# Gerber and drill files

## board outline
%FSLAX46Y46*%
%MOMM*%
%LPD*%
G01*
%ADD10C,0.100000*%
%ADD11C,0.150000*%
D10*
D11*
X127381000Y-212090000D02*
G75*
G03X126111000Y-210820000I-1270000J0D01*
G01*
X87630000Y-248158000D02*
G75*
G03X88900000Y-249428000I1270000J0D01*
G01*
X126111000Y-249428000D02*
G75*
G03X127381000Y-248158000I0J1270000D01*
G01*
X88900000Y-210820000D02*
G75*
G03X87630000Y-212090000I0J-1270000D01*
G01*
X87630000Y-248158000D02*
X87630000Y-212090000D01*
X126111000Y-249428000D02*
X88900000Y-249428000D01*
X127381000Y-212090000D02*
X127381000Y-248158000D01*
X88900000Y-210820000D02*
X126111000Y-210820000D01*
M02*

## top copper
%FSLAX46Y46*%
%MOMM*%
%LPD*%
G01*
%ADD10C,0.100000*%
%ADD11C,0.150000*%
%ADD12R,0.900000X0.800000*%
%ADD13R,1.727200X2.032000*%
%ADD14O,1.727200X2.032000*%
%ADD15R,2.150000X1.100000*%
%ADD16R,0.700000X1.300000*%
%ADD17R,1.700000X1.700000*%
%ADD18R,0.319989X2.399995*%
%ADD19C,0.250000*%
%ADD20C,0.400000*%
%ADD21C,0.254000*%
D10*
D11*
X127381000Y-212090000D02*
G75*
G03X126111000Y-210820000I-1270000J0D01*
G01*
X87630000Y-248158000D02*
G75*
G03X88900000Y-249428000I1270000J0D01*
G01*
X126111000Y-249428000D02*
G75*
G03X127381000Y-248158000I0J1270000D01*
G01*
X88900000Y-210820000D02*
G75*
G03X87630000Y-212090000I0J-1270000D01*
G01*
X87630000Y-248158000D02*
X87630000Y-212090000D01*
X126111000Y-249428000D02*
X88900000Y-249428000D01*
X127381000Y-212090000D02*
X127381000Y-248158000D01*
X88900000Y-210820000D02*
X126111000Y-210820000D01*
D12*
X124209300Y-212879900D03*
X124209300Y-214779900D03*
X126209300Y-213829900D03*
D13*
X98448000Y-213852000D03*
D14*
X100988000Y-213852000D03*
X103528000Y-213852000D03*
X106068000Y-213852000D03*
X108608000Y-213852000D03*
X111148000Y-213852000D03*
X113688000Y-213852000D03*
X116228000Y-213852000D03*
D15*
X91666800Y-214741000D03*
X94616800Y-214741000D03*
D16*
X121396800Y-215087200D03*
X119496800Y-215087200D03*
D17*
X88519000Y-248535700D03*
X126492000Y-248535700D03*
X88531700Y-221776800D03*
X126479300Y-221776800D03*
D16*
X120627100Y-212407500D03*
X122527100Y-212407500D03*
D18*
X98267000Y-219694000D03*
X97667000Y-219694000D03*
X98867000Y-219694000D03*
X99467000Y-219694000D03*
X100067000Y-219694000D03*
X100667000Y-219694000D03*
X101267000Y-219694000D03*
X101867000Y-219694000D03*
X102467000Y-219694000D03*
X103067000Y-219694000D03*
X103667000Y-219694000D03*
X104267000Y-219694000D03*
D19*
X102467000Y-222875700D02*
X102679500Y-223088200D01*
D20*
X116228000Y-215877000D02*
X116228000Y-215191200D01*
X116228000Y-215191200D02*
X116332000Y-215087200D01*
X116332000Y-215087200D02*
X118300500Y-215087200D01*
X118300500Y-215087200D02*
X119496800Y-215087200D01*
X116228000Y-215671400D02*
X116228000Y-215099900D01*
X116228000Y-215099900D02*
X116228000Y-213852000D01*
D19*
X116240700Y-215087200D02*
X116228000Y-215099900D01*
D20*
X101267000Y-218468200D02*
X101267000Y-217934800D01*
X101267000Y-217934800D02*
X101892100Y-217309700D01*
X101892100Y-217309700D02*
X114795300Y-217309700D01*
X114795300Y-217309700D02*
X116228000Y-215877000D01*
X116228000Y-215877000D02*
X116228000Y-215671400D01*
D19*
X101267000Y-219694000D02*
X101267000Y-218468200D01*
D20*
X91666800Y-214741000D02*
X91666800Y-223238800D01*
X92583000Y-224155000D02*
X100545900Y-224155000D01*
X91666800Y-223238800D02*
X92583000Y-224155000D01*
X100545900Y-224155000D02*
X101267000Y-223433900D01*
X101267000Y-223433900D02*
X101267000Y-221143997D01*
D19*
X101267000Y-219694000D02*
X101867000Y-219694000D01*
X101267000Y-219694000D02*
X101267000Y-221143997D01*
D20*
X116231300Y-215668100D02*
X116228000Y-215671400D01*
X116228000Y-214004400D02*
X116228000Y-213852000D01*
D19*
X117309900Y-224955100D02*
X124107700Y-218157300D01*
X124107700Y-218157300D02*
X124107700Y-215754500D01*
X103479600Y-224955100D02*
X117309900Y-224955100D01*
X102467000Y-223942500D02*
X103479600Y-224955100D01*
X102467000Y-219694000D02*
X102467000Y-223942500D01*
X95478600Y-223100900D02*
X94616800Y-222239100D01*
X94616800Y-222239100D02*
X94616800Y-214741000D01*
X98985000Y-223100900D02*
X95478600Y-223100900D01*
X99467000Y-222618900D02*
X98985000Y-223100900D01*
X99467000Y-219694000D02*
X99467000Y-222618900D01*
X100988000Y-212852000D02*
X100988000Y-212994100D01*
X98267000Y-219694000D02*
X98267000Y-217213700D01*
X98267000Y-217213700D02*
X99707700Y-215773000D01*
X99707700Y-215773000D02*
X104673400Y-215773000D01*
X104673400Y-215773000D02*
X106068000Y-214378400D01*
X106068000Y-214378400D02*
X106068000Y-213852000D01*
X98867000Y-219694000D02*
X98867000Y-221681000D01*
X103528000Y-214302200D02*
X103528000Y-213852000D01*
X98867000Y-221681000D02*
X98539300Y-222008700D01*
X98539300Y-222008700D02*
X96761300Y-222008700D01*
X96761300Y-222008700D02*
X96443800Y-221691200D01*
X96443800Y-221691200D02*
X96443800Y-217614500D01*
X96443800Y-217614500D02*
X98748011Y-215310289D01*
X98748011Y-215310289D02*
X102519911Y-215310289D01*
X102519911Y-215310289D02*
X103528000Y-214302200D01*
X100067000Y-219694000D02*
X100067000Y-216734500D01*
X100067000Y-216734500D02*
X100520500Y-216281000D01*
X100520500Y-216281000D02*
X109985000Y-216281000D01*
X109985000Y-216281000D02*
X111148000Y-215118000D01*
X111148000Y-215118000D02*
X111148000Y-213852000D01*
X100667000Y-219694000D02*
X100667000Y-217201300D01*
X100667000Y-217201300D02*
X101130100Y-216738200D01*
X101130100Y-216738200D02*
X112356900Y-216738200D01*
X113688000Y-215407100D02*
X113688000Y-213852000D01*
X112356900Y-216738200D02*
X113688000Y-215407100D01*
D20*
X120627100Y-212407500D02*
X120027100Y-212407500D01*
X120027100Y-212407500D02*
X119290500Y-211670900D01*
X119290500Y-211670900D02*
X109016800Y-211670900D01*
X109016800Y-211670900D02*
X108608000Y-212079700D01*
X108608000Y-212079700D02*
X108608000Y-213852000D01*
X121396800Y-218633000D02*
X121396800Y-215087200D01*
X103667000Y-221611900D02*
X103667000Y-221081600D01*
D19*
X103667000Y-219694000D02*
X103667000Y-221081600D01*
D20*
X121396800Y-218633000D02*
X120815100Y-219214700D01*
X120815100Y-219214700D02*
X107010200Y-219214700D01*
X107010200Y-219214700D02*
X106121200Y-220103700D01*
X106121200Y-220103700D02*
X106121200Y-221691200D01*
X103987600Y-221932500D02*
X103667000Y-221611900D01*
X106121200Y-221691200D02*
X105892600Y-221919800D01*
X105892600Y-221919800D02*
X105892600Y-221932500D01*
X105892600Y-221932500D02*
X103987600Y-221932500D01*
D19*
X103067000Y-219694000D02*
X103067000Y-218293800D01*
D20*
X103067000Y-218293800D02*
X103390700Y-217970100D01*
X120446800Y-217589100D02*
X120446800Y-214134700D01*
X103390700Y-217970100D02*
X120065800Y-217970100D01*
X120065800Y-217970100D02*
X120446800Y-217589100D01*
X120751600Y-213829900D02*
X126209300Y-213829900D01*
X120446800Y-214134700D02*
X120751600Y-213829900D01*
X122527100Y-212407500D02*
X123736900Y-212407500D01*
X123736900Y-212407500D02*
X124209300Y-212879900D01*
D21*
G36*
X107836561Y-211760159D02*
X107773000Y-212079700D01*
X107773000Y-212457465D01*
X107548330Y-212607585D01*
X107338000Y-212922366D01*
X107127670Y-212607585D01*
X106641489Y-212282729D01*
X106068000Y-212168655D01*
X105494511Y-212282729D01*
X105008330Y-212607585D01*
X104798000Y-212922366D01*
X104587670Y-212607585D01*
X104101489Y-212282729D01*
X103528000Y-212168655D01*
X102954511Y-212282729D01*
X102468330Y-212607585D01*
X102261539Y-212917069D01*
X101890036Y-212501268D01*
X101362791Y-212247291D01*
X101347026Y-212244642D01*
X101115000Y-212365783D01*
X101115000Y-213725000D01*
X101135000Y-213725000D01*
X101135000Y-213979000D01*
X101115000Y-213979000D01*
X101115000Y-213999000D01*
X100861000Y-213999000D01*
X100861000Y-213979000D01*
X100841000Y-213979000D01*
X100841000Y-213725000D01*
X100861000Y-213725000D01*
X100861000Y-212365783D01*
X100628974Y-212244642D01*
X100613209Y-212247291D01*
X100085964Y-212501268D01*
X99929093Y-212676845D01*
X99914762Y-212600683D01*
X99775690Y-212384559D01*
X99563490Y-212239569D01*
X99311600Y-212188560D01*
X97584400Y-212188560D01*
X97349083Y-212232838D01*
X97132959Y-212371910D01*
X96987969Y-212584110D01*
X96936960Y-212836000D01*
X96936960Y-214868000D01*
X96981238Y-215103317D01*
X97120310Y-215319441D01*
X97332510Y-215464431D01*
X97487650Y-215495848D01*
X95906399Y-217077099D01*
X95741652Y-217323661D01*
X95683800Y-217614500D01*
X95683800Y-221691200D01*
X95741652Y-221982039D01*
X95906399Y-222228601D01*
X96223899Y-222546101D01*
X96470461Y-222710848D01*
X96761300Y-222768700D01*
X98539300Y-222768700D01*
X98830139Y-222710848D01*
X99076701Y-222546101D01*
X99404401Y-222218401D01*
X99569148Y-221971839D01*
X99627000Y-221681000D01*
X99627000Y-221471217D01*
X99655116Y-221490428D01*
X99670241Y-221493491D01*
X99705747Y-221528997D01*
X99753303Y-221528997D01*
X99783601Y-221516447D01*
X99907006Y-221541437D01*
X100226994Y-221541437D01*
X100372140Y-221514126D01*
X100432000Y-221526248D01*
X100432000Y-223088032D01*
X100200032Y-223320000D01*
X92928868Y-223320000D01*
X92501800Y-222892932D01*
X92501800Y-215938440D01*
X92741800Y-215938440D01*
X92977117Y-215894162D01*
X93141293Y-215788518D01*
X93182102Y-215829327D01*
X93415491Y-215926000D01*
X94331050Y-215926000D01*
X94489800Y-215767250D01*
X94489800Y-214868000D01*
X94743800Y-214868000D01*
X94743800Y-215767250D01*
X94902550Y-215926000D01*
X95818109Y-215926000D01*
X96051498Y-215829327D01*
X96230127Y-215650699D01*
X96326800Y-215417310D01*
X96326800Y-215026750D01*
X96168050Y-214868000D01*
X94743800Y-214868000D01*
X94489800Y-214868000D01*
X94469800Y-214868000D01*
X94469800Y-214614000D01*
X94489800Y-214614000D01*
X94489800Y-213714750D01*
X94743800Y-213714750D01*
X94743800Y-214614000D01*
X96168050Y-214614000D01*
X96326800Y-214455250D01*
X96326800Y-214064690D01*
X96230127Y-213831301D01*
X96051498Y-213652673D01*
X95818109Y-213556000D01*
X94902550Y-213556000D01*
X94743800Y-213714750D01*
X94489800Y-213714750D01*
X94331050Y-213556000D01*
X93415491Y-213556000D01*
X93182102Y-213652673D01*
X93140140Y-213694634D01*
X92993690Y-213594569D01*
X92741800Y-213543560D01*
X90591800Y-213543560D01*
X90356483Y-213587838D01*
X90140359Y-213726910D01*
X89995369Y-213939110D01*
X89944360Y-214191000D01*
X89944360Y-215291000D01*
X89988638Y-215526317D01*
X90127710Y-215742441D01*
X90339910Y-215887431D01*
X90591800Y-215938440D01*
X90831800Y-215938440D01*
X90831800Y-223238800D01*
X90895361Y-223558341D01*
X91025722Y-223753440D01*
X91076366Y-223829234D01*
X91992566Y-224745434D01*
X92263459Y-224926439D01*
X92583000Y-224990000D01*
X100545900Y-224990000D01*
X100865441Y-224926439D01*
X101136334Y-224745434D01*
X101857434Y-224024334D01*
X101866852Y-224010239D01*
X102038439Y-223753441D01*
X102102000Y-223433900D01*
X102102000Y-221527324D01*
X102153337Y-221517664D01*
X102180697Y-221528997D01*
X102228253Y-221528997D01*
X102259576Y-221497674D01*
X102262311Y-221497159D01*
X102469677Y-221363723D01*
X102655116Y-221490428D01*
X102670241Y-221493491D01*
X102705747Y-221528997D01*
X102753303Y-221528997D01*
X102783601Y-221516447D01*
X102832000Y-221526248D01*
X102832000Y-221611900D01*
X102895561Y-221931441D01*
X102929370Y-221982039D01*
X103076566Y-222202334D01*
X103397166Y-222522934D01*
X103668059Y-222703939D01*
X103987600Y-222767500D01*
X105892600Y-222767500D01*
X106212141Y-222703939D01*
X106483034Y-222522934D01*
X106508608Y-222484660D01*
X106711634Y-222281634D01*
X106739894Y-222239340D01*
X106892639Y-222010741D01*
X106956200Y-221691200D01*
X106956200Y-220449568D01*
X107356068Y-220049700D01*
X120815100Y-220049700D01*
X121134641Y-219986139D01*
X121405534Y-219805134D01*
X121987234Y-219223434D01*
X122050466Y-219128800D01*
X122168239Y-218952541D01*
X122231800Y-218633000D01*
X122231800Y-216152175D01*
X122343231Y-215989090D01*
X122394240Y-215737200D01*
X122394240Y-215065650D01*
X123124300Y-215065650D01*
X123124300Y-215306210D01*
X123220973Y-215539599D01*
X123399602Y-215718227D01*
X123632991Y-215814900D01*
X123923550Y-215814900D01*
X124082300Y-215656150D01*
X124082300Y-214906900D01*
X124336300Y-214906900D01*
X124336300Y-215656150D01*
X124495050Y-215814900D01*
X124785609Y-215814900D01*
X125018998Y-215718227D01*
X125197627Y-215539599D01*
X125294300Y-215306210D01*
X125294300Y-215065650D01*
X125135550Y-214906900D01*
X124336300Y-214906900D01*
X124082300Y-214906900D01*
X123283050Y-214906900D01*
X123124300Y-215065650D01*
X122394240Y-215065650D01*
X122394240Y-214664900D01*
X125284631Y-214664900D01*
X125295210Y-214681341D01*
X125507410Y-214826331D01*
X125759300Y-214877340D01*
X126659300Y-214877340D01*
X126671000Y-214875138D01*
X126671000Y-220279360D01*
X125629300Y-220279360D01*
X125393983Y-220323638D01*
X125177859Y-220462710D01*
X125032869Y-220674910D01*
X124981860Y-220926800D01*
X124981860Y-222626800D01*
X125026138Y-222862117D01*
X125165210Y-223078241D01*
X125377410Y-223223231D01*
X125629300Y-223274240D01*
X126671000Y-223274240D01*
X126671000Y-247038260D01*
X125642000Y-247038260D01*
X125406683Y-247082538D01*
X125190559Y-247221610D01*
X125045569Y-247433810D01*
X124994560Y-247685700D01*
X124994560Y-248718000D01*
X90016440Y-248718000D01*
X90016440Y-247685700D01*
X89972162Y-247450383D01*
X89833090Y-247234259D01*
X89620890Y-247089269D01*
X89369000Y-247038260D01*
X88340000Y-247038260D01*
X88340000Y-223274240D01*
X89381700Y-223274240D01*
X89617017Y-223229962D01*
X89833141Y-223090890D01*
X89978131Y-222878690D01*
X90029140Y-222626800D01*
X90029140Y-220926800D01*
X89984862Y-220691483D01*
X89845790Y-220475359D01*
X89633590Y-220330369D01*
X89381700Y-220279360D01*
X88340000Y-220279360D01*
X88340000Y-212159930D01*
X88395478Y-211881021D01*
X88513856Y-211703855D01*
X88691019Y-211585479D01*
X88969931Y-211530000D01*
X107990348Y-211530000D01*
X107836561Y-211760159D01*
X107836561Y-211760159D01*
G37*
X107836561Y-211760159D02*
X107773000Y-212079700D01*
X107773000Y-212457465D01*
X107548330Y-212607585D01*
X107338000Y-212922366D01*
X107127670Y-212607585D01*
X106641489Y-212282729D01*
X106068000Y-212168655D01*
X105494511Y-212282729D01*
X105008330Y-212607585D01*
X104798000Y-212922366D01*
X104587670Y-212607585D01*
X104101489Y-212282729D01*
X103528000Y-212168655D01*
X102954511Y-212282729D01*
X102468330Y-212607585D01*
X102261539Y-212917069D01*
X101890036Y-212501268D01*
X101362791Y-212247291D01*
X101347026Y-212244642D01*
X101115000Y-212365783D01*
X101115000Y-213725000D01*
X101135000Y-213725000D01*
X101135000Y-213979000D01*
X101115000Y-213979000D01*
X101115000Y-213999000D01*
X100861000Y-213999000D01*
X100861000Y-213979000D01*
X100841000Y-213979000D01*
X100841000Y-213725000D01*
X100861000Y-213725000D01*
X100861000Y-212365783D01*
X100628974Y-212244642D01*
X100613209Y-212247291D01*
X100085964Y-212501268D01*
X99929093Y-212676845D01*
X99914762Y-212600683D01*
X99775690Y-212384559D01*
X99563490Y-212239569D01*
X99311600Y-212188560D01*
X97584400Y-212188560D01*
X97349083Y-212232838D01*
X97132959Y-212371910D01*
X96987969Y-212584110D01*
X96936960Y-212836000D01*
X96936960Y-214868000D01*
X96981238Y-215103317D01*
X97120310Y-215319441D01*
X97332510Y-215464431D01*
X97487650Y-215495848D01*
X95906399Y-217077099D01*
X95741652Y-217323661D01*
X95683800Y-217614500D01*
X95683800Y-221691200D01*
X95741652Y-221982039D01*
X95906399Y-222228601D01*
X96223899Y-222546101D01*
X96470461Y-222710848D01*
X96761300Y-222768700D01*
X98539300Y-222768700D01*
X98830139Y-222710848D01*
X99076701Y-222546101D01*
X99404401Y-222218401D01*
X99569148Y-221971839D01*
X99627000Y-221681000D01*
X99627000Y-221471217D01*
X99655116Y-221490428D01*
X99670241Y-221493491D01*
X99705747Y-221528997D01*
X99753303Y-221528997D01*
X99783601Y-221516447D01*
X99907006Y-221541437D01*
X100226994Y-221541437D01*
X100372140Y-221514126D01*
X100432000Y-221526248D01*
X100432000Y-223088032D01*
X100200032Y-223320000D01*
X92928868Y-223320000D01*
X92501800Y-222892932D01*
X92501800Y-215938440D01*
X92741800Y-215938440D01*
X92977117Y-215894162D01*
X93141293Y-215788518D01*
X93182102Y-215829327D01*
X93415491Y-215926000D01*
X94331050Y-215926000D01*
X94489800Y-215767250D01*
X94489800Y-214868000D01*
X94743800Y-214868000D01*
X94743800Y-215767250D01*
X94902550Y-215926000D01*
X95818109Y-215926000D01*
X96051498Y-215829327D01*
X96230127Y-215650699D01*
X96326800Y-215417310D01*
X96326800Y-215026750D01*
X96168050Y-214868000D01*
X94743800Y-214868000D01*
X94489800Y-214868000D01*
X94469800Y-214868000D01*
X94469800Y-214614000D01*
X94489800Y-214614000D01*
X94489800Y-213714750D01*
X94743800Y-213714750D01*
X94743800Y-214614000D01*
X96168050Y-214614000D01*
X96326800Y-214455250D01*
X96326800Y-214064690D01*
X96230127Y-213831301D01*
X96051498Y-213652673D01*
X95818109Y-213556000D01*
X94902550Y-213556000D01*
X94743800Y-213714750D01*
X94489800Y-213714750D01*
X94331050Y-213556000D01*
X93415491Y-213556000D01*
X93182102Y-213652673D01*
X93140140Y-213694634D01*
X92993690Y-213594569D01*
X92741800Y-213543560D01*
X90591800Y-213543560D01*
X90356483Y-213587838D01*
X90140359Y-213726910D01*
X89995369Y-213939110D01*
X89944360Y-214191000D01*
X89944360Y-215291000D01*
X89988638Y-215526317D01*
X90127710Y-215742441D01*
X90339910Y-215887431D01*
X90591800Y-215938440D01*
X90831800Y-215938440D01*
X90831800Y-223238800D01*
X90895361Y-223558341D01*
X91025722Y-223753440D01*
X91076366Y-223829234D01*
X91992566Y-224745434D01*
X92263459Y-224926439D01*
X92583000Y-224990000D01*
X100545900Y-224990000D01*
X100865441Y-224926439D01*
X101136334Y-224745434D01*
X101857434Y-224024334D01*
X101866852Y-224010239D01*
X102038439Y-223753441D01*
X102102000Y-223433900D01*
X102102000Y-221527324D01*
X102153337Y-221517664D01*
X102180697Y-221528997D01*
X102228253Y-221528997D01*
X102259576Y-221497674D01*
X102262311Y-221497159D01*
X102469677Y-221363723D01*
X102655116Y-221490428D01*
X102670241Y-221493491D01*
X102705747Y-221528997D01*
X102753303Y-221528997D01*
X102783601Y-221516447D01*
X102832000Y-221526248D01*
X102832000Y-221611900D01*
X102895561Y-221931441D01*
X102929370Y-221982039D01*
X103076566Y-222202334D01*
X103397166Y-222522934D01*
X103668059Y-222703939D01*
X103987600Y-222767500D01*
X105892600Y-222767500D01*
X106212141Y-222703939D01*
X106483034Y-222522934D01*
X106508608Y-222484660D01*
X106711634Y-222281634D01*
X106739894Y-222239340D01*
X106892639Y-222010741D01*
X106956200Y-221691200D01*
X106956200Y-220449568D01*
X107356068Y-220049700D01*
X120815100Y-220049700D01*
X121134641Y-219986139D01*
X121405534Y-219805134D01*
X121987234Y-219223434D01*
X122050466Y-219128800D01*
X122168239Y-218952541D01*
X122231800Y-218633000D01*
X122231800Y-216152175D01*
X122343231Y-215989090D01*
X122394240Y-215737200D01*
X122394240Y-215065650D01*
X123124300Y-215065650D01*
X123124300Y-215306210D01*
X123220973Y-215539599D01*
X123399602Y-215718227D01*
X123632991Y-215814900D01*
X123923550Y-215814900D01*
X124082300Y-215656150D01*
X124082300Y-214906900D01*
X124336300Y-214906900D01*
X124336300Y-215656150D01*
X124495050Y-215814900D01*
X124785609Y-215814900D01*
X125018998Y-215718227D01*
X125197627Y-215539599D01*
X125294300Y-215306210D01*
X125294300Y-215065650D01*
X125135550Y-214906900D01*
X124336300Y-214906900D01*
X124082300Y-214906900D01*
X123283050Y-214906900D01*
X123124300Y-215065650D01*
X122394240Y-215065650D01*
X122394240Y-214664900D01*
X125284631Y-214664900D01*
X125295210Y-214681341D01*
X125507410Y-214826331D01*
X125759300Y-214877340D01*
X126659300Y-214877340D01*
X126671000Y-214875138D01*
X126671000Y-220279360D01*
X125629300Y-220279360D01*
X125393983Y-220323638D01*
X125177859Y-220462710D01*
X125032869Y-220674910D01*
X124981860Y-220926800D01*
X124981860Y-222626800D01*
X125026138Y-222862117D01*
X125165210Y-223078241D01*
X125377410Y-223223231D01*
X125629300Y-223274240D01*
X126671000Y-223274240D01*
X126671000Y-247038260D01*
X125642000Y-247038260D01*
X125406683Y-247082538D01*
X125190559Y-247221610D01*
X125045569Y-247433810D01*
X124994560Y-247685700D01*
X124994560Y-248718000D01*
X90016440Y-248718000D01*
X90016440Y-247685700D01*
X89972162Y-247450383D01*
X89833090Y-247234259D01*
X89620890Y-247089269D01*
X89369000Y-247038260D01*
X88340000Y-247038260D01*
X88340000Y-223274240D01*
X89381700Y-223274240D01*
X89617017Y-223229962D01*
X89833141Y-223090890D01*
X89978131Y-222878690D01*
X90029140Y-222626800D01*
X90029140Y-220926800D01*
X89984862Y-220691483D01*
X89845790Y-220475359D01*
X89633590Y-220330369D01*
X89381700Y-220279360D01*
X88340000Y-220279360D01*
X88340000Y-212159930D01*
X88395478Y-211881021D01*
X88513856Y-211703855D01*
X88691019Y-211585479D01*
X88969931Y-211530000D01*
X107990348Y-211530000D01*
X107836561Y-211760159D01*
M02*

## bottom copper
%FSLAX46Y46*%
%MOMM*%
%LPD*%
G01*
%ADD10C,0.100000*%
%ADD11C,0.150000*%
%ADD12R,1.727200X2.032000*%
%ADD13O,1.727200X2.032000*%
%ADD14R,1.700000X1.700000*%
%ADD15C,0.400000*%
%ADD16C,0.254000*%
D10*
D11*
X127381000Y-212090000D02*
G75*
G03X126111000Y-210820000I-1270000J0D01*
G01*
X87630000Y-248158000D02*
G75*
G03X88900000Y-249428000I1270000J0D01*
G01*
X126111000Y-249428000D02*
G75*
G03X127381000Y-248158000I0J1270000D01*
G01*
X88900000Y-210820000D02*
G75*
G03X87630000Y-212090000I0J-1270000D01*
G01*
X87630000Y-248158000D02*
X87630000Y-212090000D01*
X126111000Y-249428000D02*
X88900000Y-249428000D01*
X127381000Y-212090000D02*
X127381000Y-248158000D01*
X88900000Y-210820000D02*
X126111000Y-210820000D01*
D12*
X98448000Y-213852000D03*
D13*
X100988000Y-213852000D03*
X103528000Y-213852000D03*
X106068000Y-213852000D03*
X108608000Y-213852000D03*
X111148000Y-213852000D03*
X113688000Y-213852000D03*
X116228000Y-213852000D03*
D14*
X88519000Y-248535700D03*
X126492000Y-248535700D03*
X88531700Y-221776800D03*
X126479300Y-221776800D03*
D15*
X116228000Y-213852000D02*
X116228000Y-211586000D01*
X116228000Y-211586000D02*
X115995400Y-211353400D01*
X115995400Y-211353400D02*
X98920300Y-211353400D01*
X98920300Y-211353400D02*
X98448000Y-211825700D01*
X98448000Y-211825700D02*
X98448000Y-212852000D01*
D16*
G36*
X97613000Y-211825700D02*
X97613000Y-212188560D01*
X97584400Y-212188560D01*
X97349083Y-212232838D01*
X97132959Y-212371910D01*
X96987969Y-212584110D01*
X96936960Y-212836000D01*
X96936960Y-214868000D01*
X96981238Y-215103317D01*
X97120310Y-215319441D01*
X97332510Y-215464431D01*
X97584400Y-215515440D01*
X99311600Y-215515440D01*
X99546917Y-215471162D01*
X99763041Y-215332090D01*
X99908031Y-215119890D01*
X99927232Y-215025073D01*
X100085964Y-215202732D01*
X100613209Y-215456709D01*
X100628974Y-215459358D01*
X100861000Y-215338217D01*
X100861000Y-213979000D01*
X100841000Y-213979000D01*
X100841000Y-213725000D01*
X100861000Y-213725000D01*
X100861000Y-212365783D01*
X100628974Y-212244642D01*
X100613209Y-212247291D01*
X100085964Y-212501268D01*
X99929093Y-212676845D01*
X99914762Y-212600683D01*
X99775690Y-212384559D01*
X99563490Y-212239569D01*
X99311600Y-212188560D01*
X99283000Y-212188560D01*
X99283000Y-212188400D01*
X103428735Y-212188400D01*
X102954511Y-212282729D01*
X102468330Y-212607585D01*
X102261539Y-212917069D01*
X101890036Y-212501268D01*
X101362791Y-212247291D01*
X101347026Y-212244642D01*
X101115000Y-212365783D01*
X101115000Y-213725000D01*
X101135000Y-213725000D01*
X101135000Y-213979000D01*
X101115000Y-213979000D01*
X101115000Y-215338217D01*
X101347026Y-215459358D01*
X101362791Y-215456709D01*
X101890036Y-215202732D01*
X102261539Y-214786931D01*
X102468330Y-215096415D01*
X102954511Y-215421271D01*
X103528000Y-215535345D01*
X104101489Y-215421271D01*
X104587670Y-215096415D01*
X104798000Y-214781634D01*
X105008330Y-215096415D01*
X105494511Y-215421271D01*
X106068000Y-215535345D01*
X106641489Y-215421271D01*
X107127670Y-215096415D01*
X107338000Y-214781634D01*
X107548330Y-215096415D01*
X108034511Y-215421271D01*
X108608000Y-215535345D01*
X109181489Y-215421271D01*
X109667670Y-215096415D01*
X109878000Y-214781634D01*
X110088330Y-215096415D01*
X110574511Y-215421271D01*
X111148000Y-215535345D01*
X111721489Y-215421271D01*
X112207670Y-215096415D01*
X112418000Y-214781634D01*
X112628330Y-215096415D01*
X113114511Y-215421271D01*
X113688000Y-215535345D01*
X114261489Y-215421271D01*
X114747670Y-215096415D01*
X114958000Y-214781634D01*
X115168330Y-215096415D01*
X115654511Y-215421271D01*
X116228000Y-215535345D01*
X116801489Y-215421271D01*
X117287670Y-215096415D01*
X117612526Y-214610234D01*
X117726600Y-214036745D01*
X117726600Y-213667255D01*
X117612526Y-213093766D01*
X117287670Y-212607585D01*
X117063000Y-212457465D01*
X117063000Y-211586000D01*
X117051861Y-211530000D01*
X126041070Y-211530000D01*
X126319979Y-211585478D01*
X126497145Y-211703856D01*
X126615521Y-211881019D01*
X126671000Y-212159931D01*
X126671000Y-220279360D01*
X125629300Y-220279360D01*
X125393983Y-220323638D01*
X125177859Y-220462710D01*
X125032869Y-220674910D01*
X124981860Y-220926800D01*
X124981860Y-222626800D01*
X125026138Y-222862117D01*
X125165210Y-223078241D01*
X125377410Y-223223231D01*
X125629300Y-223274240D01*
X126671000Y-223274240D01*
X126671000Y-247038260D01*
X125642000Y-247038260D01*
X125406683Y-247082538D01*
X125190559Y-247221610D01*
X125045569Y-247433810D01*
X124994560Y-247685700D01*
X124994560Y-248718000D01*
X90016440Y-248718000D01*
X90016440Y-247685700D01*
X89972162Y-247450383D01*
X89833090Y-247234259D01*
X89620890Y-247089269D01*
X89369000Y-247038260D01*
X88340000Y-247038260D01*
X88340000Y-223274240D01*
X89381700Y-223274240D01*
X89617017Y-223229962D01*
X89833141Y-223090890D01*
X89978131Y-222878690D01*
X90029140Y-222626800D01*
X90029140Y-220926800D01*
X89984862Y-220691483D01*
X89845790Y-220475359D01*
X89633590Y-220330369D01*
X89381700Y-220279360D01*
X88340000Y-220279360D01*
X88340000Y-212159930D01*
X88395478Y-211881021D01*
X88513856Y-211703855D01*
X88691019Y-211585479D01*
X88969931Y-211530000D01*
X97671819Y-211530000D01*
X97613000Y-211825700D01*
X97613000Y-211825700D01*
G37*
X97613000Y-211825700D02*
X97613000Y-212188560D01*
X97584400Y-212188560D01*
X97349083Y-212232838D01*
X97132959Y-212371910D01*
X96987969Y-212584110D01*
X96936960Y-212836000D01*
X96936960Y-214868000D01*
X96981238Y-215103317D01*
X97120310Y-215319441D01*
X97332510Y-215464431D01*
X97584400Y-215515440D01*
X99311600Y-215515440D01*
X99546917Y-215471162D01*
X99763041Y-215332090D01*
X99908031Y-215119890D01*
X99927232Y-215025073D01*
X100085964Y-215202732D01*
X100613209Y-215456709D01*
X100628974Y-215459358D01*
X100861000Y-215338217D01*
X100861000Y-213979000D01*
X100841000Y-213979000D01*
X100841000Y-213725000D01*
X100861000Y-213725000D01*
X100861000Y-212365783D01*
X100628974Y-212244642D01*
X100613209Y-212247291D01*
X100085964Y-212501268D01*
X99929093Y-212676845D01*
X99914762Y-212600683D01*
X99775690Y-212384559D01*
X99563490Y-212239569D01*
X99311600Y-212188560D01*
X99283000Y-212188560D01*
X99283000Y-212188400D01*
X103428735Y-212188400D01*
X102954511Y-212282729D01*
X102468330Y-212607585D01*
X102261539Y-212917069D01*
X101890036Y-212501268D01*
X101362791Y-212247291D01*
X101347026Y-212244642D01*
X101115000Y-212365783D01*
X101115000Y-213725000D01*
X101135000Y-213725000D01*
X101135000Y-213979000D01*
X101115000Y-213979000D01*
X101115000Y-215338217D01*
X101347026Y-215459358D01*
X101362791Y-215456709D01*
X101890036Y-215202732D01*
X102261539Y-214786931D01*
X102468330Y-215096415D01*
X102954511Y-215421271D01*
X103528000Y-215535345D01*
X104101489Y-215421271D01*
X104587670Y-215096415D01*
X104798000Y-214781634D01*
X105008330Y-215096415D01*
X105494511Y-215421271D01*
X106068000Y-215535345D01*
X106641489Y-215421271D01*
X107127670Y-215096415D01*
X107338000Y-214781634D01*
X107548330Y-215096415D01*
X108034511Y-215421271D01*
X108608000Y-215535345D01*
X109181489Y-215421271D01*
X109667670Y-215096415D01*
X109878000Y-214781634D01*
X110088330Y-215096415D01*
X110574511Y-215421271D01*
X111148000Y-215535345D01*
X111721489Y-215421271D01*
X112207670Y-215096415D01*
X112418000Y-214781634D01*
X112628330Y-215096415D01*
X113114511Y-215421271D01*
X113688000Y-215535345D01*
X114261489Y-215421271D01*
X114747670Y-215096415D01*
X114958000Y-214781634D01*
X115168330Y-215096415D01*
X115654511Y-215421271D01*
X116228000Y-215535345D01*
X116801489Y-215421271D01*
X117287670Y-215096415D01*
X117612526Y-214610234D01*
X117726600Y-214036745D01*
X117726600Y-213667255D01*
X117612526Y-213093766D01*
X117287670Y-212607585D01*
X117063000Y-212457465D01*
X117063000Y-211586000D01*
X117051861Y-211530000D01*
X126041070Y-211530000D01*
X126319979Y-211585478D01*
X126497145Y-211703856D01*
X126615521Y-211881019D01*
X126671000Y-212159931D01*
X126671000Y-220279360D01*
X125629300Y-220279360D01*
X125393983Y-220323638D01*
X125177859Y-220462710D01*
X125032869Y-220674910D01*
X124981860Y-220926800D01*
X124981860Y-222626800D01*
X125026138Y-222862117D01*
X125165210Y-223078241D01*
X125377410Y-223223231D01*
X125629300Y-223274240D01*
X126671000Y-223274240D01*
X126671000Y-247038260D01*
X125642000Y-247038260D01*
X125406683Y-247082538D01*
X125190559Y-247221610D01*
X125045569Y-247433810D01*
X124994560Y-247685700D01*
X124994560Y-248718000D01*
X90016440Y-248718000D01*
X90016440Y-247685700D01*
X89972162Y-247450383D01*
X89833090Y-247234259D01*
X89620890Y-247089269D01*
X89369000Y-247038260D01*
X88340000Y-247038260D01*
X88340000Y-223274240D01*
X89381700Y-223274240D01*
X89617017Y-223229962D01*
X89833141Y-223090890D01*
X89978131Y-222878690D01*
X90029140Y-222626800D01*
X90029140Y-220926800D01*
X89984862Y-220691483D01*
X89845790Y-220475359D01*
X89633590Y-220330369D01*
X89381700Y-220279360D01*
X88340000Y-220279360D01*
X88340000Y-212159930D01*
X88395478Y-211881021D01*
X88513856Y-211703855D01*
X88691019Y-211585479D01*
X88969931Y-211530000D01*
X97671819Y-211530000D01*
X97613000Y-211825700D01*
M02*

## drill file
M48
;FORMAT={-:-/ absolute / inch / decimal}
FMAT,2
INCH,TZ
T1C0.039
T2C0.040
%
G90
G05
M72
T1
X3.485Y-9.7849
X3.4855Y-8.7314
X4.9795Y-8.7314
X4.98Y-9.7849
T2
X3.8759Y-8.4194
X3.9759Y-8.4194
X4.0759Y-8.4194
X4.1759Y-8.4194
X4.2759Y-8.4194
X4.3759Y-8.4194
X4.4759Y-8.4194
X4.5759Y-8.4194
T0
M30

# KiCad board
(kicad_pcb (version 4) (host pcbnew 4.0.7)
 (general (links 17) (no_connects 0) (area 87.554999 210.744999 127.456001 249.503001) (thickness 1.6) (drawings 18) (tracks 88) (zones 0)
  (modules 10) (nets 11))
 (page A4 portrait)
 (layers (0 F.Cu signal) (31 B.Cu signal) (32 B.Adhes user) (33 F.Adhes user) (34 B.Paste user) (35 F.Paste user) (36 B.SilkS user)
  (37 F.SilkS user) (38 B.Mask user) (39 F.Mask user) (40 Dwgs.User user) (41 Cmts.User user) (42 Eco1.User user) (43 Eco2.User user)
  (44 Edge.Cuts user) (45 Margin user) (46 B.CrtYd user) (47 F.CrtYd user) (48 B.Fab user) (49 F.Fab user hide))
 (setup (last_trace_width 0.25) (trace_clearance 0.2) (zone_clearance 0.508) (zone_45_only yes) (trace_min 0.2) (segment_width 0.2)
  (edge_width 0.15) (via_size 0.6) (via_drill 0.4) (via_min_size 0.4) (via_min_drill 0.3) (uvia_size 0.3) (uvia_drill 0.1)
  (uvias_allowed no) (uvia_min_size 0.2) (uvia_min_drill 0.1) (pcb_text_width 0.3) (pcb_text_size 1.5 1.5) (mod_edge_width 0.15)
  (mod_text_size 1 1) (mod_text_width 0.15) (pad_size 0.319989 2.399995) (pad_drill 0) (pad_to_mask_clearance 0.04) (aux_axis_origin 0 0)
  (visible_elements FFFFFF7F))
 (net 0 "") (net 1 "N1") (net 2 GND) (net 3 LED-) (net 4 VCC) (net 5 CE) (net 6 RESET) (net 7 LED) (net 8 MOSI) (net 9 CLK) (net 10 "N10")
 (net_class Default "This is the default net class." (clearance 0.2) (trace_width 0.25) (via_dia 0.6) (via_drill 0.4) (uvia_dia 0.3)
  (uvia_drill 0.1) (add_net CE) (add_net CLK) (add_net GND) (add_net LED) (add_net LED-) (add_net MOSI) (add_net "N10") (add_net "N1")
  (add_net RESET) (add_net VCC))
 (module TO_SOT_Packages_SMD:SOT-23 (layer F.Cu) (at 125.2093 213.8299)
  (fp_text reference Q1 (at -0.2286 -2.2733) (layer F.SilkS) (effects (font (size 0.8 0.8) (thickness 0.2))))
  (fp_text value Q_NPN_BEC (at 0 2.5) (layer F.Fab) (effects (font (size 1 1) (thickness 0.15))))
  (pad 1 smd rect (at -1 -0.95) (size 0.9 0.8) (layers F.Cu F.Paste F.Mask) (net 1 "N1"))
  (pad 2 smd rect (at -1 0.95) (size 0.9 0.8) (layers F.Cu F.Paste F.Mask) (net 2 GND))
  (pad 3 smd rect (at 1 0) (size 0.9 0.8) (layers F.Cu F.Paste F.Mask) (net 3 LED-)))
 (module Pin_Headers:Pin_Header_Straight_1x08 (layer F.Cu) (at 98.448 213.852 90)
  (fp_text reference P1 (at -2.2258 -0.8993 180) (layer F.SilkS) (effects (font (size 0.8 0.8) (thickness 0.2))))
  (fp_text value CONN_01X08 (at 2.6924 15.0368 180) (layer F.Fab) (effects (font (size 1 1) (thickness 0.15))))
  (pad 1 thru_hole rect (at 0 0 90) (size 2.032 1.7272) (drill 1.016) (layers *.Cu *.Mask F.SilkS) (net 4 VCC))
  (pad 2 thru_hole oval (at 0 2.54 90) (size 2.032 1.7272) (drill 1.016) (layers *.Cu *.Mask F.SilkS) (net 2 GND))
  (pad 3 thru_hole oval (at 0 5.08 90) (size 2.032 1.7272) (drill 1.016) (layers *.Cu *.Mask F.SilkS) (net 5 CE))
  (pad 4 thru_hole oval (at 0 7.62 90) (size 2.032 1.7272) (drill 1.016) (layers *.Cu *.Mask F.SilkS) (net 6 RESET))
  (pad 5 thru_hole oval (at 0 10.16 90) (size 2.032 1.7272) (drill 1.016) (layers *.Cu *.Mask F.SilkS) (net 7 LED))
  (pad 6 thru_hole oval (at 0 12.7 90) (size 2.032 1.7272) (drill 1.016) (layers *.Cu *.Mask F.SilkS) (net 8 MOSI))
  (pad 7 thru_hole oval (at 0 15.24 90) (size 2.032 1.7272) (drill 1.016) (layers *.Cu *.Mask F.SilkS) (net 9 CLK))
  (pad 8 thru_hole oval (at 0 17.78 90) (size 2.032 1.7272) (drill 1.016) (layers *.Cu *.Mask F.SilkS) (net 4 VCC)))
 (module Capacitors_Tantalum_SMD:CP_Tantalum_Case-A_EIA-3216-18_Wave (layer F.Cu) (at 93.1418 214.741)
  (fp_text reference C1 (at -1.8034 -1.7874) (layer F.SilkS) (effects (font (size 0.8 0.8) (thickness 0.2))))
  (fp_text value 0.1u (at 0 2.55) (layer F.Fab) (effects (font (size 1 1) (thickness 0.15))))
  (pad 1 smd rect (at -1.475 0) (size 2.15 1.1) (layers F.Cu F.Paste F.Mask) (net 4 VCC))
  (pad 2 smd rect (at 1.475 0) (size 2.15 1.1) (layers F.Cu F.Paste F.Mask) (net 2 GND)))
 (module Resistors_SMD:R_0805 (layer F.Cu) (at 120.4468 215.0872 180)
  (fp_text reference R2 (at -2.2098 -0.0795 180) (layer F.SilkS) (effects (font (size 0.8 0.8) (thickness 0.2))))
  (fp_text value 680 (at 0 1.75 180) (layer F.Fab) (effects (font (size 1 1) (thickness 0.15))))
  (pad 1 smd rect (at -0.95 0 180) (size 0.7 1.3) (layers F.Cu F.Paste F.Mask) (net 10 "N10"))
  (pad 2 smd rect (at 0.95 0 180) (size 0.7 1.3) (layers F.Cu F.Paste F.Mask) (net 4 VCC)))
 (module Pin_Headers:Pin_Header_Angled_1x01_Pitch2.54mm (layer F.Cu) (at 88.519 248.5357)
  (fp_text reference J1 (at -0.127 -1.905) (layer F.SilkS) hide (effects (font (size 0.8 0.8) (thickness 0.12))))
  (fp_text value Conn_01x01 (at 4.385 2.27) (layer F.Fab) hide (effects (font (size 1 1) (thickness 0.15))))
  (pad 1 thru_hole rect (at 0 0) (size 1.7 1.7) (drill 1) (layers *.Cu *.Mask)))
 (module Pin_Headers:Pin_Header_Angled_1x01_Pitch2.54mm (layer F.Cu) (at 126.492 248.5357 180)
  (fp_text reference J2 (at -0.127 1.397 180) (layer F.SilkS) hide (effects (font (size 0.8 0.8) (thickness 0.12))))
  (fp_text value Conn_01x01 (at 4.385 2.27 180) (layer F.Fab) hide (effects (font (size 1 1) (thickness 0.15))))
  (pad 1 thru_hole rect (at 0 0 180) (size 1.7 1.7) (drill 1) (layers *.Cu *.Mask)))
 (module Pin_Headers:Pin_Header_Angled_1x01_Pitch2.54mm (layer F.Cu) (at 88.5317 221.7768)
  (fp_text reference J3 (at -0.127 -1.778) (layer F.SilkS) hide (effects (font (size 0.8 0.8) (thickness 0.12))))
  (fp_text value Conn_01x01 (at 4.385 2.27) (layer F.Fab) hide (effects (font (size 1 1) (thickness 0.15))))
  (pad 1 thru_hole rect (at 0 0) (size 1.7 1.7) (drill 1) (layers *.Cu *.Mask)))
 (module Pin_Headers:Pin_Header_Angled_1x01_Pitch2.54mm (layer F.Cu) (at 126.4793 221.7768 180)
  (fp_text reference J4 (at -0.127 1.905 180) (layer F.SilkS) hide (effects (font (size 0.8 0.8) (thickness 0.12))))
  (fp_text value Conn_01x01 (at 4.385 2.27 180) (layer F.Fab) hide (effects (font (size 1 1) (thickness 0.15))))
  (pad 1 thru_hole rect (at 0 0 180) (size 1.7 1.7) (drill 1) (layers *.Cu *.Mask)))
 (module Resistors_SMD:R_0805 (layer F.Cu) (at 121.5771 212.4075)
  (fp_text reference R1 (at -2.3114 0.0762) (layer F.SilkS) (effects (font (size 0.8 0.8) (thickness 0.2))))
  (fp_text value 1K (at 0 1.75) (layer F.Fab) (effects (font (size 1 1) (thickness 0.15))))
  (pad 1 smd rect (at -0.95 0) (size 0.7 1.3) (layers F.Cu F.Paste F.Mask) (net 7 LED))
  (pad 2 smd rect (at 0.95 0) (size 0.7 1.3) (layers F.Cu F.Paste F.Mask) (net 1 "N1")))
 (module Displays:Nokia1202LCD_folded (layer F.Cu) (at 100.969 219.694)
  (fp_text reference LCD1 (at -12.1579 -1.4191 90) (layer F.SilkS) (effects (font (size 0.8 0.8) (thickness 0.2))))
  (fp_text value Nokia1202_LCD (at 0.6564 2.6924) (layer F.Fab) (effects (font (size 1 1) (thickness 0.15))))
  (pad 2 smd rect (at -2.702 0) (size 0.319989 2.399995) (layers F.Cu F.Paste F.Mask) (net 6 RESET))
  (pad 1 smd rect (at -3.302 0) (size 0.319989 2.399995) (layers F.Cu F.Paste F.Mask))
  (pad 3 smd rect (at -2.102 0) (size 0.319989 2.399995) (layers F.Cu F.Paste F.Mask) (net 5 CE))
  (pad 4 smd rect (at -1.502 0) (size 0.319989 2.399995) (layers F.Cu F.Paste F.Mask) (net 2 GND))
  (pad 5 smd rect (at -0.902 0) (size 0.319989 2.399995) (layers F.Cu F.Paste F.Mask) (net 8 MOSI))
  (pad 6 smd rect (at -0.302 0) (size 0.319989 2.399995) (layers F.Cu F.Paste F.Mask) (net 9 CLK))
  (pad 7 smd rect (at 0.298 0) (size 0.319989 2.399995) (layers F.Cu F.Paste F.Mask) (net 4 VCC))
  (pad 8 smd rect (at 0.898 0) (size 0.319989 2.399995) (layers F.Cu F.Paste F.Mask) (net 4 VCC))
  (pad 9 smd rect (at 1.498 0) (size 0.319989 2.399995) (layers F.Cu F.Paste F.Mask) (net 2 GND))
  (pad 10 smd rect (at 2.098 0) (size 0.319989 2.399995) (layers F.Cu F.Paste F.Mask) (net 3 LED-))
  (pad 11 smd rect (at 2.698 0) (size 0.319989 2.399995) (layers F.Cu F.Paste F.Mask) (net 10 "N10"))
  (pad 12 smd rect (at 3.298 0) (size 0.319989 2.399995) (layers F.Cu F.Paste F.Mask)))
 (gr_arc (start 126.111 212.09) (end 126.111 210.82) (angle 90) (layer Edge.Cuts) (width 0.15))
 (gr_arc (start 88.9 248.158) (end 88.9 249.428) (angle 90) (layer Edge.Cuts) (width 0.15))
 (gr_arc (start 126.111 248.158) (end 127.381 248.158) (angle 90) (layer Edge.Cuts) (width 0.15))
 (gr_arc (start 88.9 212.09) (end 87.63 212.09) (angle 90) (layer Edge.Cuts) (width 0.15))
 (gr_line (start 87.63 248.158) (end 87.63 212.09) (layer Edge.Cuts) (width 0.15))
 (gr_line (start 126.111 249.428) (end 88.9 249.428) (layer Edge.Cuts) (width 0.15))
 (gr_line (start 127.381 212.09) (end 127.381 248.158) (layer Edge.Cuts) (width 0.15))
 (gr_line (start 88.9 210.82) (end 126.111 210.82) (layer Edge.Cuts) (width 0.15))
 (segment (start 102.467 222.8757) (end 102.6795 223.0882) (width 0.25) (layer F.Cu) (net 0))
 (segment (start 116.228 215.877) (end 116.228 215.1912) (width 0.4) (layer F.Cu) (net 4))
 (segment (start 116.228 215.1912) (end 116.332 215.0872) (width 0.4) (layer F.Cu) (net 4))
 (segment (start 116.332 215.0872) (end 118.3005 215.0872) (width 0.4) (layer F.Cu) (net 4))
 (segment (start 118.3005 215.0872) (end 119.4968 215.0872) (width 0.4) (layer F.Cu) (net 4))
 (segment (start 116.228 215.6714) (end 116.228 215.0999) (width 0.4) (layer F.Cu) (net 4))
 (segment (start 116.228 215.0999) (end 116.228 213.852) (width 0.4) (layer F.Cu) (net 4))
 (segment (start 116.2407 215.0872) (end 116.228 215.0999) (width 0.25) (layer F.Cu) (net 4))
 (segment (start 101.267 218.4682) (end 101.267 217.9348) (width 0.4) (layer F.Cu) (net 4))
 (segment (start 101.267 217.9348) (end 101.8921 217.3097) (width 0.4) (layer F.Cu) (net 4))
 (segment (start 101.8921 217.3097) (end 114.7953 217.3097) (width 0.4) (layer F.Cu) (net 4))
 (segment (start 114.7953 217.3097) (end 116.228 215.877) (width 0.4) (layer F.Cu) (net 4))
 (segment (start 116.228 215.877) (end 116.228 215.6714) (width 0.4) (layer F.Cu) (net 4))
 (segment (start 101.267 219.694) (end 101.267 218.4682) (width 0.25) (layer F.Cu) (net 4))
 (segment (start 91.6668 214.741) (end 91.6668 223.2388) (width 0.4) (layer F.Cu) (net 4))
 (segment (start 92.583 224.155) (end 100.5459 224.155) (width 0.4) (layer F.Cu) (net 4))
 (segment (start 91.6668 223.2388) (end 92.583 224.155) (width 0.4) (layer F.Cu) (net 4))
 (segment (start 100.5459 224.155) (end 101.267 223.4339) (width 0.4) (layer F.Cu) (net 4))
 (segment (start 101.267 223.4339) (end 101.267 221.143997) (width 0.4) (layer F.Cu) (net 4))
 (segment (start 101.267 219.694) (end 101.867 219.694) (width 0.25) (layer F.Cu) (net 4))
 (segment (start 101.267 219.694) (end 101.267 221.143997) (width 0.25) (layer F.Cu) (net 4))
 (segment (start 116.228 213.852) (end 116.228 211.586) (width 0.4) (layer B.Cu) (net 4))
 (segment (start 116.228 211.586) (end 115.9954 211.3534) (width 0.4) (layer B.Cu) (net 4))
 (segment (start 115.9954 211.3534) (end 98.9203 211.3534) (width 0.4) (layer B.Cu) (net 4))
 (segment (start 98.9203 211.3534) (end 98.448 211.8257) (width 0.4) (layer B.Cu) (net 4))
 (segment (start 98.448 211.8257) (end 98.448 212.852) (width 0.4) (layer B.Cu) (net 4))
 (segment (start 116.2313 215.6681) (end 116.228 215.6714) (width 0.4) (layer F.Cu) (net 4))
 (segment (start 116.228 214.0044) (end 116.228 213.852) (width 0.4) (layer F.Cu) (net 4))
 (segment (start 117.3099 224.9551) (end 124.1077 218.1573) (width 0.25) (layer F.Cu) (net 2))
 (segment (start 124.1077 218.1573) (end 124.1077 215.7545) (width 0.25) (layer F.Cu) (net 2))
 (segment (start 103.4796 224.9551) (end 117.3099 224.9551) (width 0.25) (layer F.Cu) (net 2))
 (segment (start 102.467 223.9425) (end 103.4796 224.9551) (width 0.25) (layer F.Cu) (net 2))
 (segment (start 102.467 219.694) (end 102.467 223.9425) (width 0.25) (layer F.Cu) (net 2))
 (segment (start 95.4786 223.1009) (end 94.6168 222.2391) (width 0.25) (layer F.Cu) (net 2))
 (segment (start 94.6168 222.2391) (end 94.6168 214.741) (width 0.25) (layer F.Cu) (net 2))
 (segment (start 98.985 223.1009) (end 95.4786 223.1009) (width 0.25) (layer F.Cu) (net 2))
 (segment (start 99.467 222.6189) (end 98.985 223.1009) (width 0.25) (layer F.Cu) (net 2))
 (segment (start 99.467 219.694) (end 99.467 222.6189) (width 0.25) (layer F.Cu) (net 2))
 (segment (start 100.988 212.852) (end 100.988 212.9941) (width 0.25) (layer F.Cu) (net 2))
 (segment (start 98.267 219.694) (end 98.267 217.2137) (width 0.25) (layer F.Cu) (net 6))
 (segment (start 98.267 217.2137) (end 99.7077 215.773) (width 0.25) (layer F.Cu) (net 6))
 (segment (start 99.7077 215.773) (end 104.6734 215.773) (width 0.25) (layer F.Cu) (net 6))
 (segment (start 104.6734 215.773) (end 106.068 214.3784) (width 0.25) (layer F.Cu) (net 6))
 (segment (start 106.068 214.3784) (end 106.068 213.852) (width 0.25) (layer F.Cu) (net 6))
 (segment (start 98.867 219.694) (end 98.867 221.681) (width 0.25) (layer F.Cu) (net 5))
 (segment (start 103.528 214.3022) (end 103.528 213.852) (width 0.25) (layer F.Cu) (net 5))
 (segment (start 98.867 221.681) (end 98.5393 222.0087) (width 0.25) (layer F.Cu) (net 5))
 (segment (start 98.5393 222.0087) (end 96.7613 222.0087) (width 0.25) (layer F.Cu) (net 5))
 (segment (start 96.7613 222.0087) (end 96.4438 221.6912) (width 0.25) (layer F.Cu) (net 5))
 (segment (start 96.4438 221.6912) (end 96.4438 217.6145) (width 0.25) (layer F.Cu) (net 5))
 (segment (start 96.4438 217.6145) (end 98.748011 215.310289) (width 0.25) (layer F.Cu) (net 5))
 (segment (start 98.748011 215.310289) (end 102.519911 215.310289) (width 0.25) (layer F.Cu) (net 5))
 (segment (start 102.519911 215.310289) (end 103.528 214.3022) (width 0.25) (layer F.Cu) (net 5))
 (segment (start 100.067 219.694) (end 100.067 216.7345) (width 0.25) (layer F.Cu) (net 8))
 (segment (start 100.067 216.7345) (end 100.5205 216.281) (width 0.25) (layer F.Cu) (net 8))
 (segment (start 100.5205 216.281) (end 109.985 216.281) (width 0.25) (layer F.Cu) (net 8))
 (segment (start 109.985 216.281) (end 111.148 215.118) (width 0.25) (layer F.Cu) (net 8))
 (segment (start 111.148 215.118) (end 111.148 213.852) (width 0.25) (layer F.Cu) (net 8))
 (segment (start 100.667 219.694) (end 100.667 217.2013) (width 0.25) (layer F.Cu) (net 9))
 (segment (start 100.667 217.2013) (end 101.1301 216.7382) (width 0.25) (layer F.Cu) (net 9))
 (segment (start 101.1301 216.7382) (end 112.3569 216.7382) (width 0.25) (layer F.Cu) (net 9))
 (segment (start 113.688 215.4071) (end 113.688 213.852) (width 0.25) (layer F.Cu) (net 9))
 (segment (start 112.3569 216.7382) (end 113.688 215.4071) (width 0.25) (layer F.Cu) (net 9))
 (segment (start 120.6271 212.4075) (end 120.0271 212.4075) (width 0.4) (layer F.Cu) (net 7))
 (segment (start 120.0271 212.4075) (end 119.2905 211.6709) (width 0.4) (layer F.Cu) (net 7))
 (segment (start 119.2905 211.6709) (end 109.0168 211.6709) (width 0.4) (layer F.Cu) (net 7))
 (segment (start 109.0168 211.6709) (end 108.608 212.0797) (width 0.4) (layer F.Cu) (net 7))
 (segment (start 108.608 212.0797) (end 108.608 213.852) (width 0.4) (layer F.Cu) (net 7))
 (segment (start 121.3968 218.633) (end 121.3968 215.0872) (width 0.4) (layer F.Cu) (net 10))
 (segment (start 103.667 221.6119) (end 103.667 221.0816) (width 0.4) (layer F.Cu) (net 10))
 (segment (start 103.667 219.694) (end 103.667 221.0816) (width 0.25) (layer F.Cu) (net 10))
 (segment (start 121.3968 218.633) (end 120.8151 219.2147) (width 0.4) (layer F.Cu) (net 10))
 (segment (start 120.8151 219.2147) (end 107.0102 219.2147) (width 0.4) (layer F.Cu) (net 10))
 (segment (start 107.0102 219.2147) (end 106.1212 220.1037) (width 0.4) (layer F.Cu) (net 10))
 (segment (start 106.1212 220.1037) (end 106.1212 221.6912) (width 0.4) (layer F.Cu) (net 10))
 (segment (start 103.9876 221.9325) (end 103.667 221.6119) (width 0.4) (layer F.Cu) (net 10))
 (segment (start 106.1212 221.6912) (end 105.8926 221.9198) (width 0.4) (layer F.Cu) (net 10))
 (segment (start 105.8926 221.9198) (end 105.8926 221.9325) (width 0.4) (layer F.Cu) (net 10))
 (segment (start 105.8926 221.9325) (end 103.9876 221.9325) (width 0.4) (layer F.Cu) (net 10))
 (segment (start 103.067 219.694) (end 103.067 218.2938) (width 0.25) (layer F.Cu) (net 3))
 (segment (start 103.067 218.2938) (end 103.3907 217.9701) (width 0.4) (layer F.Cu) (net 3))
 (segment (start 120.4468 217.5891) (end 120.4468 214.1347) (width 0.4) (layer F.Cu) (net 3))
 (segment (start 103.3907 217.9701) (end 120.0658 217.9701) (width 0.4) (layer F.Cu) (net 3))
 (segment (start 120.0658 217.9701) (end 120.4468 217.5891) (width 0.4) (layer F.Cu) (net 3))
 (segment (start 120.7516 213.8299) (end 126.2093 213.8299) (width 0.4) (layer F.Cu) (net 3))
 (segment (start 120.4468 214.1347) (end 120.7516 213.8299) (width 0.4) (layer F.Cu) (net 3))
 (segment (start 122.5271 212.4075) (end 123.7369 212.4075) (width 0.4) (layer F.Cu) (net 1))
 (segment (start 123.7369 212.4075) (end 124.2093 212.8799) (width 0.4) (layer F.Cu) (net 1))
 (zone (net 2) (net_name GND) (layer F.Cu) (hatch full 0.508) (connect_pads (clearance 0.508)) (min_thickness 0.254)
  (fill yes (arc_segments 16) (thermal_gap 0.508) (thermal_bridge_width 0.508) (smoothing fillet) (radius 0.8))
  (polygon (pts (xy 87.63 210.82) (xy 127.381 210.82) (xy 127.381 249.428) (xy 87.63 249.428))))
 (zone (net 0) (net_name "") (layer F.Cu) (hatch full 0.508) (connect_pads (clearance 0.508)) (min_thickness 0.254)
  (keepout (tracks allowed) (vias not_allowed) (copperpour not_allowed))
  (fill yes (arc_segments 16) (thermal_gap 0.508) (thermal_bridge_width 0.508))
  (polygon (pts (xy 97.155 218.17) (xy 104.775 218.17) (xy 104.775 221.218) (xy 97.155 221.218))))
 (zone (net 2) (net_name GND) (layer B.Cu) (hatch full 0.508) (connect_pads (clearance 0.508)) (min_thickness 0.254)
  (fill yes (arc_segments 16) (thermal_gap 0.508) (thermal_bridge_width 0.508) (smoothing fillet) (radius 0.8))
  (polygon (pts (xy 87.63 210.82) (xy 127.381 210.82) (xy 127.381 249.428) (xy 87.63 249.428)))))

